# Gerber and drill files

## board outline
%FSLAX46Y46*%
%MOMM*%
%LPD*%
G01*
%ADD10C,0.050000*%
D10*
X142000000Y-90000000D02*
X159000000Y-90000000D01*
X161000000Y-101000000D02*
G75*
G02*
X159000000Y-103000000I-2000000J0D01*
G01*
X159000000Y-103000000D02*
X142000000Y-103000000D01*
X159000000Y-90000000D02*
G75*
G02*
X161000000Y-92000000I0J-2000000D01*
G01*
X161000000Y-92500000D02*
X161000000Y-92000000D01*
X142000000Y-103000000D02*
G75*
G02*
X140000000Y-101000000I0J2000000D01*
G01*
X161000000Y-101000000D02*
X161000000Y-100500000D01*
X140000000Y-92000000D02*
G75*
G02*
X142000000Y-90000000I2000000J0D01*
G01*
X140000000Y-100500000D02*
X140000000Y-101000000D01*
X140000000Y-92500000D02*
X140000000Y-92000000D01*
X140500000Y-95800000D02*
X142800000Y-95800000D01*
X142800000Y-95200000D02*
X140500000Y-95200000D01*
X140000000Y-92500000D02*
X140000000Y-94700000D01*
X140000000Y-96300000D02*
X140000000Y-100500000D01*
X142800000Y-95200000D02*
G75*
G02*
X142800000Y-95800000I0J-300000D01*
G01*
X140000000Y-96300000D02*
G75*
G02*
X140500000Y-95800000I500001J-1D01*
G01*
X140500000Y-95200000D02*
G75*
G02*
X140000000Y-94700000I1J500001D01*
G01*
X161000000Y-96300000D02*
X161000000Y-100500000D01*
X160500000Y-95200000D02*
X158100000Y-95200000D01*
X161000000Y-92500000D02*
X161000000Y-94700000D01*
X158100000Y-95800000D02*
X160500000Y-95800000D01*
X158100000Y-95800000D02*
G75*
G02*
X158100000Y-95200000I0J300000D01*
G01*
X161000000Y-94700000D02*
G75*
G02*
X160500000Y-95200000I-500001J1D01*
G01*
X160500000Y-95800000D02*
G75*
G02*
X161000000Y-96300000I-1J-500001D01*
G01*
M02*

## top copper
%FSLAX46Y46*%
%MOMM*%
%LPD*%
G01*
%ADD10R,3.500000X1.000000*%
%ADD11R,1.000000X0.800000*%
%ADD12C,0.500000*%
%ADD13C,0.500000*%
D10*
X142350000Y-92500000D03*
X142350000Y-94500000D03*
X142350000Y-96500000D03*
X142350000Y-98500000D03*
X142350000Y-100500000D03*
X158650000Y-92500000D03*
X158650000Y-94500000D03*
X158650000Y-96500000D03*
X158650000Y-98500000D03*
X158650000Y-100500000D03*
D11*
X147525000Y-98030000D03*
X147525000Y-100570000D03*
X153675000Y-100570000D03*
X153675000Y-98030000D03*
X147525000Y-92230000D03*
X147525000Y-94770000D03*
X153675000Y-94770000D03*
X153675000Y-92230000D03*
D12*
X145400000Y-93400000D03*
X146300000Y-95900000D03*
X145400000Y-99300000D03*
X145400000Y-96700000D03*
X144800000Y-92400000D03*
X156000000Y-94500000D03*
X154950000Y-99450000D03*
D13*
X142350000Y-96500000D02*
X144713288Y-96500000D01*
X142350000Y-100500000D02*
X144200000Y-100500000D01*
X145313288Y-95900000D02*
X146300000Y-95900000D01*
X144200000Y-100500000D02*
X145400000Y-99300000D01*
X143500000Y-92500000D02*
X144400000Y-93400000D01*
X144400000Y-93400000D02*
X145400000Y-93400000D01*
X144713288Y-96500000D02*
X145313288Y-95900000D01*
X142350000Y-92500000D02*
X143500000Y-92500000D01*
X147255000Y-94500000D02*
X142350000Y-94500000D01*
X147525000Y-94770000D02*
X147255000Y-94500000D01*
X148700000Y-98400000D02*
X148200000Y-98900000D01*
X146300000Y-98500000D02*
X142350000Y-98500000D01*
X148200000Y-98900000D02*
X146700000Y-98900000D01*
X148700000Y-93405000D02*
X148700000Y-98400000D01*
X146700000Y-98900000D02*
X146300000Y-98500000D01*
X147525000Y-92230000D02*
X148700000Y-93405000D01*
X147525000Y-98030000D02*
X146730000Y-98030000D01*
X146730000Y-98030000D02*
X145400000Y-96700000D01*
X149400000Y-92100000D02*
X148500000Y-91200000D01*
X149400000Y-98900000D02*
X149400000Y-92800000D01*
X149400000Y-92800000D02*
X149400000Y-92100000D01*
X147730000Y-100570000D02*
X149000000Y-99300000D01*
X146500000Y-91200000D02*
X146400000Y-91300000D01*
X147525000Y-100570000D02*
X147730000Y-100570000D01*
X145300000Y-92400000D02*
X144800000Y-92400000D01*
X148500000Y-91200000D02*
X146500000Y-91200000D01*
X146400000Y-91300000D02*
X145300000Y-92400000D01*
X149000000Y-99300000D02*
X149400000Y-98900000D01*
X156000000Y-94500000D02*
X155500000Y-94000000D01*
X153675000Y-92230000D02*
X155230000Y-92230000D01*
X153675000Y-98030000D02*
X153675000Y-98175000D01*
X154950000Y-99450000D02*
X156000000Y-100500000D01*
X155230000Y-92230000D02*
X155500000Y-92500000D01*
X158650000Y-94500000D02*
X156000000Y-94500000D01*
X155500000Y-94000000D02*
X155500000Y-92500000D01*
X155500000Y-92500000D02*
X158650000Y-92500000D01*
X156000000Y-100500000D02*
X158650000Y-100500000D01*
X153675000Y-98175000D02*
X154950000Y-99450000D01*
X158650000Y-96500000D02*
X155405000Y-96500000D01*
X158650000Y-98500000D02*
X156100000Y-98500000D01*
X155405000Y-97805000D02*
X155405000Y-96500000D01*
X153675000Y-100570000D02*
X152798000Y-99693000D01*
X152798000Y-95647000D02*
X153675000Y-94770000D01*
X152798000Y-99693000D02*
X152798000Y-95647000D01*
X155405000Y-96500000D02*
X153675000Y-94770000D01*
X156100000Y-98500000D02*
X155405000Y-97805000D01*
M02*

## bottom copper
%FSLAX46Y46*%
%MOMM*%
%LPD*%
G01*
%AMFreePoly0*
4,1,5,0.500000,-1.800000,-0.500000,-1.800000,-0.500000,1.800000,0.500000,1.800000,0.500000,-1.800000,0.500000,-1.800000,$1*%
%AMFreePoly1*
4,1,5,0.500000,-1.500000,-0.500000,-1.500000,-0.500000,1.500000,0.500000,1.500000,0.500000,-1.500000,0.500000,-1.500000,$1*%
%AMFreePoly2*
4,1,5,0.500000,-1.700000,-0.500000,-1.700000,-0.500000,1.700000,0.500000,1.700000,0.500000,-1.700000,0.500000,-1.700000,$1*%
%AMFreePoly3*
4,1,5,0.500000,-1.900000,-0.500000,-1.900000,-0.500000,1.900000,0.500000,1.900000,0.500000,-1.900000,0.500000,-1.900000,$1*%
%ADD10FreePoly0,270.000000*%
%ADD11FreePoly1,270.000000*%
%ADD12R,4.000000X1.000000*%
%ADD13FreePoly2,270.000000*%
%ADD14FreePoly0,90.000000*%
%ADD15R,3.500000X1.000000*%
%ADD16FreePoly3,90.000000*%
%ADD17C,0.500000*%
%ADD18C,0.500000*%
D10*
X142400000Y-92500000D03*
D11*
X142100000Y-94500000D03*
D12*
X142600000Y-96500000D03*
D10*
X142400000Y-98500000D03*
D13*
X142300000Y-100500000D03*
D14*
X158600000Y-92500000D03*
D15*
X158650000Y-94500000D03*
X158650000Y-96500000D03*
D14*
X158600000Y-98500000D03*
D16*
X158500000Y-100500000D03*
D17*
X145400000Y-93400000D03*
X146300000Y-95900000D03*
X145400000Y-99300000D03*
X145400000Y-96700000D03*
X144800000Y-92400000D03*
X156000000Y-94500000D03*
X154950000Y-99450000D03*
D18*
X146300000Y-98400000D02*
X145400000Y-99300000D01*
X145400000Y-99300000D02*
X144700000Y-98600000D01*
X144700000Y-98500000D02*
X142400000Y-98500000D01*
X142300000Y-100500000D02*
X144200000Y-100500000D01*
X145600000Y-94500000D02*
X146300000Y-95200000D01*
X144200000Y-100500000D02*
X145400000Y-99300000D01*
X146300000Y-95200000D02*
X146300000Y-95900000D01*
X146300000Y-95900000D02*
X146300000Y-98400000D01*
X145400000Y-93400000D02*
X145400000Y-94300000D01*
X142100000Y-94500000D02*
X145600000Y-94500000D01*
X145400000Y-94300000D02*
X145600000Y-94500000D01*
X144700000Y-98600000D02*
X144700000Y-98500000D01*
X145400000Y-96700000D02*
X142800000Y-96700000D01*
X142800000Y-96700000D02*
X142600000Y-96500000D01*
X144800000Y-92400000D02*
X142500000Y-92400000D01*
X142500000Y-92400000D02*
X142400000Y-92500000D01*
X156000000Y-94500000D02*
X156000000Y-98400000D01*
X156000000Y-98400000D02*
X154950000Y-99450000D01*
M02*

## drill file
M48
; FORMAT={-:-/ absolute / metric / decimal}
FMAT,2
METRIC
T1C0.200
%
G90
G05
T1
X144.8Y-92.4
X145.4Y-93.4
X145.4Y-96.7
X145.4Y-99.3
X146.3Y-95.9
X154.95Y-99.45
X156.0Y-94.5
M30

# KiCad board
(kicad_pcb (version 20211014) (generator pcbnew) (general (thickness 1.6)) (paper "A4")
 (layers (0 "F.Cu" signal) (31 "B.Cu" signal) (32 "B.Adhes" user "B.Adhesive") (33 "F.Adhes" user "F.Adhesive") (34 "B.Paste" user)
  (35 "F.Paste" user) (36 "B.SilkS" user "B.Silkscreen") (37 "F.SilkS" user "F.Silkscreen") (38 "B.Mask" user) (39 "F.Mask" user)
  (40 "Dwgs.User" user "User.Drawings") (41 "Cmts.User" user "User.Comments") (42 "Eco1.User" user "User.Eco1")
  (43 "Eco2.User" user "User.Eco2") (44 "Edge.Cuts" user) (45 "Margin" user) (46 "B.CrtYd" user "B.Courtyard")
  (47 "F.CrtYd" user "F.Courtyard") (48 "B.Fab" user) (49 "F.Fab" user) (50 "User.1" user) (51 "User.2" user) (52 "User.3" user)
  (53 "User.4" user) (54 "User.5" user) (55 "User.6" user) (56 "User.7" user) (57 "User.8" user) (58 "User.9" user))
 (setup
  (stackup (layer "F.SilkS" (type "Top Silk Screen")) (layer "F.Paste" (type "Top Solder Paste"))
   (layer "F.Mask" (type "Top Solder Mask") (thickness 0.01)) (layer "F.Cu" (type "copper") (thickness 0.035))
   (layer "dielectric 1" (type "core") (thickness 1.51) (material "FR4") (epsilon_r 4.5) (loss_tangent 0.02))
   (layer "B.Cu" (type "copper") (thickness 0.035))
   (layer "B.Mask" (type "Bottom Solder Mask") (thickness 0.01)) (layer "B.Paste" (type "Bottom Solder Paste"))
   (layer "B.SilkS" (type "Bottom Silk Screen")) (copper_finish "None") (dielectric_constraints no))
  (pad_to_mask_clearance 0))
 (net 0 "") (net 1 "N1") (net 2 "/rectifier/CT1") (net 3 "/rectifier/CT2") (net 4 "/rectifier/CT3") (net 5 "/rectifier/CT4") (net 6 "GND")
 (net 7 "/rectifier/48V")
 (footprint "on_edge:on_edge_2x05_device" (layer "F.Cu") (at 140 96.5 -90)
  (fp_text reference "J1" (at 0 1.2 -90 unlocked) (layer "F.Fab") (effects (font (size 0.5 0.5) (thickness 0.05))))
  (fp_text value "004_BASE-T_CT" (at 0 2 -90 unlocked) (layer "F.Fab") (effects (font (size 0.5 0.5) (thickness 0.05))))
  (fp_line (start -0.7 -0.5) (end -0.7 -2.8) (layer "Edge.Cuts") (width 0.05))
  (fp_line (start -1.3 -2.8) (end -1.3 -0.5) (layer "Edge.Cuts") (width 0.05))
  (fp_line (start -4 0) (end -1.8 0) (layer "Edge.Cuts") (width 0.05))
  (fp_line (start -0.2 0) (end 4 0) (layer "Edge.Cuts") (width 0.05))
  (fp_arc (start -1.3 -2.8) (mid -1 -3.1) (end -0.7 -2.8) (layer "Edge.Cuts") (width 0.05))
  (fp_arc (start -0.2 0) (mid -0.553553 -0.146447) (end -0.7 -0.5) (layer "Edge.Cuts") (width 0.05))
  (fp_arc (start -1.3 -0.5) (mid -1.446447 -0.146447) (end -1.8 0) (layer "Edge.Cuts") (width 0.05))
  (pad "1" smd rect (at -4 -2.35 90) (size 1 3.5) (layers "F.Cu" "F.Mask") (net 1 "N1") (zone_connect 0))
  (pad "2" smd rect (at -2 -2.35 270) (size 1 3.5) (layers "F.Cu" "F.Mask") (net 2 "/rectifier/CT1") (zone_connect 0))
  (pad "3" smd rect (at 0 -2.35 270) (size 1 3.5) (layers "F.Cu" "F.Mask") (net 1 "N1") (zone_connect 0))
  (pad "4" smd rect (at 2 -2.35 90) (size 1 3.5) (layers "F.Cu" "F.Mask") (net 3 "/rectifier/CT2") (zone_connect 0))
  (pad "5" smd rect (at 4 -2.35 90) (size 1 3.5) (layers "F.Cu" "F.Mask") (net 1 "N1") (zone_connect 0))
  (pad "6" smd custom (at -4 -2.4 270) (size 1 3.6) (layers "B.Cu" "B.Mask") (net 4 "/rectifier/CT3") (zone_connect 0)
   (options (clearance outline) (anchor rect)) (primitives))
  (pad "7" smd custom (at -2 -2.1 270) (size 1 3) (layers "B.Cu" "B.Mask") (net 1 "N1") (zone_connect 0)
   (options (clearance outline) (anchor rect)) (primitives))
  (pad "8" smd rect (at 0 -2.6 270) (size 1 4) (layers "B.Cu" "B.Mask") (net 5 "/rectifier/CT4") (zone_connect 0))
  (pad "9" smd custom (at 2 -2.4 270) (size 1 3.6) (layers "B.Cu" "B.Mask") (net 1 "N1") (zone_connect 0)
   (options (clearance outline) (anchor rect)) (primitives))
  (pad "10" smd custom (at 4 -2.3 270) (size 1 3.4) (layers "B.Cu" "B.Mask") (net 1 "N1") (zone_connect 0)
   (options (clearance outline) (anchor rect)) (primitives)))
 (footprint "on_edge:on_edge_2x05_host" (layer "F.Cu") (at 161 96.5 -90)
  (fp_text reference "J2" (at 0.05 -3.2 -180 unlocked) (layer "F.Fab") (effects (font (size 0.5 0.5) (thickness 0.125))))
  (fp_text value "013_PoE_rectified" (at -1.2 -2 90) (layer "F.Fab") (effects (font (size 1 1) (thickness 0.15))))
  (fp_line (start -0.2 0) (end 4 0) (layer "Edge.Cuts") (width 0.05))
  (fp_line (start -1.3 0.5) (end -1.3 2.9) (layer "Edge.Cuts") (width 0.05))
  (fp_line (start -4 0) (end -1.8 0) (layer "Edge.Cuts") (width 0.05))
  (fp_line (start -0.7 2.9) (end -0.7 0.5) (layer "Edge.Cuts") (width 0.05))
  (fp_arc (start -0.7 2.9) (mid -1 3.2) (end -1.3 2.9) (layer "Edge.Cuts") (width 0.05))
  (fp_arc (start -1.8 0) (mid -1.446447 0.146447) (end -1.3 0.5) (layer "Edge.Cuts") (width 0.05))
  (fp_arc (start -0.7 0.5) (mid -0.553553 0.146447) (end -0.2 0) (layer "Edge.Cuts") (width 0.05))
  (pad "1" smd rect (at -4 2.35 270) (size 1 3.5) (layers "F.Cu" "F.Mask") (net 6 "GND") (zone_connect 0))
  (pad "2" smd rect (at -2 2.35 270) (size 1 3.5) (layers "F.Cu" "F.Mask") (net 6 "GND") (zone_connect 0))
  (pad "3" smd rect (at 0 2.35 270) (size 1 3.5) (layers "F.Cu" "F.Mask") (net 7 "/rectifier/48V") (zone_connect 0))
  (pad "4" smd rect (at 2 2.35 270) (size 1 3.5) (layers "F.Cu" "F.Mask") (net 7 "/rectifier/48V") (zone_connect 0))
  (pad "5" smd rect (at 4 2.35 270) (size 1 3.5) (layers "F.Cu" "F.Mask") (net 6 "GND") (zone_connect 0))
  (pad "6" smd custom (at -4 2.4 90) (size 1 3.6) (layers "B.Cu" "B.Mask") (zone_connect 0) (options (clearance outline) (anchor rect))
   (primitives))
  (pad "7" smd rect (at -2 2.35 90) (size 1 3.5) (layers "B.Cu" "B.Mask") (zone_connect 0))
  (pad "8" smd rect (at 0 2.35 90) (size 1 3.5) (layers "B.Cu" "B.Mask") (zone_connect 0))
  (pad "9" smd custom (at 2 2.4 90) (size 1 3.6) (layers "B.Cu" "B.Mask") (zone_connect 0) (options (clearance outline) (anchor rect))
   (primitives))
  (pad "10" smd custom (at 4 2.5 90) (size 1 3.8) (layers "B.Cu" "B.Mask") (zone_connect 0) (options (clearance outline) (anchor rect))
   (primitives)))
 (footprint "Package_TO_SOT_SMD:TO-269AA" (layer "F.Cu") (at 150.6 99.3)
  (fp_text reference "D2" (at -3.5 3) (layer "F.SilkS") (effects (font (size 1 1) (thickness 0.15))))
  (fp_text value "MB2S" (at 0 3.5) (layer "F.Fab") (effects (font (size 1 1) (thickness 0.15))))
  (pad "1" smd rect (at -3.075 -1.27) (size 1 0.8) (layers "F.Cu" "F.Paste" "F.Mask") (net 5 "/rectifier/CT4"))
  (pad "2" smd rect (at -3.075 1.27) (size 1 0.8) (layers "F.Cu" "F.Paste" "F.Mask") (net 4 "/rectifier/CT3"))
  (pad "3" smd rect (at 3.075 1.27) (size 1 0.8) (layers "F.Cu" "F.Paste" "F.Mask") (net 7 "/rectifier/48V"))
  (pad "4" smd rect (at 3.075 -1.27) (size 1 0.8) (layers "F.Cu" "F.Paste" "F.Mask") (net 6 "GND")))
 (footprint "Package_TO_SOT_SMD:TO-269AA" (layer "F.Cu") (at 150.6 93.5)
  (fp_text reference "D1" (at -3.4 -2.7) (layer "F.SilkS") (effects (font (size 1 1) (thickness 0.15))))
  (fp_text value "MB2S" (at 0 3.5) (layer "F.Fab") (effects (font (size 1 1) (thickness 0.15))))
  (pad "1" smd rect (at -3.075 -1.27) (size 1 0.8) (layers "F.Cu" "F.Paste" "F.Mask") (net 3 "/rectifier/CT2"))
  (pad "2" smd rect (at -3.075 1.27) (size 1 0.8) (layers "F.Cu" "F.Paste" "F.Mask") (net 2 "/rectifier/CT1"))
  (pad "3" smd rect (at 3.075 1.27) (size 1 0.8) (layers "F.Cu" "F.Paste" "F.Mask") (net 7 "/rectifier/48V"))
  (pad "4" smd rect (at 3.075 -1.27) (size 1 0.8) (layers "F.Cu" "F.Paste" "F.Mask") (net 6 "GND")))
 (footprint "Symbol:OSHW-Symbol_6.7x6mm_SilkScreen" (layer "B.Cu") (at 150 99 180)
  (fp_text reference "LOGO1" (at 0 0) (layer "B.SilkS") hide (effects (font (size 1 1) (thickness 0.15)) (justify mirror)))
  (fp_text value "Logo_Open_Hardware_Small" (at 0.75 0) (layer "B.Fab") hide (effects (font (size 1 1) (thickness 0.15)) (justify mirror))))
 (gr_line (start 142 90) (end 159 90) (layer "Edge.Cuts") (width 0.05))
 (gr_arc (start 161 101) (mid 160.414214 102.414214) (end 159 103) (layer "Edge.Cuts") (width 0.05))
 (gr_line (start 159 103) (end 142 103) (layer "Edge.Cuts") (width 0.05))
 (gr_arc (start 159 90) (mid 160.414214 90.585786) (end 161 92) (layer "Edge.Cuts") (width 0.05))
 (gr_line (start 161 92.5) (end 161 92) (layer "Edge.Cuts") (width 0.05))
 (gr_arc (start 142 103) (mid 140.585786 102.414214) (end 140 101) (layer "Edge.Cuts") (width 0.05))
 (gr_line (start 161 101) (end 161 100.5) (layer "Edge.Cuts") (width 0.05))
 (gr_arc (start 140 92) (mid 140.585786 90.585786) (end 142 90) (layer "Edge.Cuts") (width 0.05))
 (gr_line (start 140 100.5) (end 140 101) (layer "Edge.Cuts") (width 0.05))
 (gr_line (start 140 92.5) (end 140 92) (layer "Edge.Cuts") (width 0.05))
 (segment (start 142.35 96.5) (end 144.713288 96.5) (width 0.5) (layer "F.Cu") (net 1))
 (segment (start 142.35 100.5) (end 144.2 100.5) (width 0.5) (layer "F.Cu") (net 1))
 (segment (start 145.313288 95.9) (end 146.3 95.9) (width 0.5) (layer "F.Cu") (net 1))
 (segment (start 144.2 100.5) (end 145.4 99.3) (width 0.5) (layer "F.Cu") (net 1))
 (segment (start 143.5 92.5) (end 144.4 93.4) (width 0.5) (layer "F.Cu") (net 1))
 (segment (start 144.4 93.4) (end 145.4 93.4) (width 0.5) (layer "F.Cu") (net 1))
 (segment (start 144.713288 96.5) (end 145.313288 95.9) (width 0.5) (layer "F.Cu") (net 1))
 (segment (start 142.35 92.5) (end 143.5 92.5) (width 0.5) (layer "F.Cu") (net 1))
 (via (at 145.4 93.4) (size 0.5) (drill 0.2) (layers "F.Cu" "B.Cu") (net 1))
 (via (at 146.3 95.9) (size 0.5) (drill 0.2) (layers "F.Cu" "B.Cu") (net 1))
 (via (at 145.4 99.3) (size 0.5) (drill 0.2) (layers "F.Cu" "B.Cu") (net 1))
 (segment (start 146.3 98.4) (end 145.4 99.3) (width 0.5) (layer "B.Cu") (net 1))
 (segment (start 145.4 99.3) (end 144.7 98.6) (width 0.5) (layer "B.Cu") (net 1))
 (segment (start 144.7 98.5) (end 142.4 98.5) (width 0.5) (layer "B.Cu") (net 1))
 (segment (start 142.3 100.5) (end 144.2 100.5) (width 0.5) (layer "B.Cu") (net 1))
 (segment (start 145.6 94.5) (end 146.3 95.2) (width 0.5) (layer "B.Cu") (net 1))
 (segment (start 144.2 100.5) (end 145.4 99.3) (width 0.5) (layer "B.Cu") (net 1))
 (segment (start 146.3 95.2) (end 146.3 95.9) (width 0.5) (layer "B.Cu") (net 1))
 (segment (start 146.3 95.9) (end 146.3 98.4) (width 0.5) (layer "B.Cu") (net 1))
 (segment (start 145.4 93.4) (end 145.4 94.3) (width 0.5) (layer "B.Cu") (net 1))
 (segment (start 142.1 94.5) (end 145.6 94.5) (width 0.5) (layer "B.Cu") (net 1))
 (segment (start 145.4 94.3) (end 145.6 94.5) (width 0.5) (layer "B.Cu") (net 1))
 (segment (start 144.7 98.6) (end 144.7 98.5) (width 0.5) (layer "B.Cu") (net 1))
 (segment (start 147.255 94.5) (end 142.35 94.5) (width 0.5) (layer "F.Cu") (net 2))
 (segment (start 147.525 94.77) (end 147.255 94.5) (width 0.5) (layer "F.Cu") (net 2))
 (segment (start 148.7 98.4) (end 148.2 98.9) (width 0.5) (layer "F.Cu") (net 3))
 (segment (start 146.3 98.5) (end 142.35 98.5) (width 0.5) (layer "F.Cu") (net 3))
 (segment (start 148.2 98.9) (end 146.7 98.9) (width 0.5) (layer "F.Cu") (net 3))
 (segment (start 148.7 93.405) (end 148.7 98.4) (width 0.5) (layer "F.Cu") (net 3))
 (segment (start 146.7 98.9) (end 146.3 98.5) (width 0.5) (layer "F.Cu") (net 3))
 (segment (start 147.525 92.23) (end 148.7 93.405) (width 0.5) (layer "F.Cu") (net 3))
 (segment (start 147.525 98.03) (end 146.73 98.03) (width 0.5) (layer "F.Cu") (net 5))
 (segment (start 146.73 98.03) (end 145.4 96.7) (width 0.5) (layer "F.Cu") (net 5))
 (via (at 145.4 96.7) (size 0.5) (drill 0.2) (layers "F.Cu" "B.Cu") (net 5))
 (segment (start 145.4 96.7) (end 142.8 96.7) (width 0.5) (layer "B.Cu") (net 5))
 (segment (start 142.8 96.7) (end 142.6 96.5) (width 0.5) (layer "B.Cu") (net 5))
 (segment (start 149.4 92.1) (end 148.5 91.2) (width 0.5) (layer "F.Cu") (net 4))
 (segment (start 149.4 98.9) (end 149.4 92.8) (width 0.5) (layer "F.Cu") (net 4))
 (segment (start 149.4 92.8) (end 149.4 92.1) (width 0.5) (layer "F.Cu") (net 4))
 (segment (start 147.73 100.57) (end 149 99.3) (width 0.5) (layer "F.Cu") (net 4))
 (segment (start 146.5 91.2) (end 146.4 91.3) (width 0.5) (layer "F.Cu") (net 4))
 (segment (start 147.525 100.57) (end 147.73 100.57) (width 0.5) (layer "F.Cu") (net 4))
 (segment (start 145.3 92.4) (end 144.8 92.4) (width 0.5) (layer "F.Cu") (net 4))
 (segment (start 148.5 91.2) (end 146.5 91.2) (width 0.5) (layer "F.Cu") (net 4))
 (segment (start 146.4 91.3) (end 145.3 92.4) (width 0.5) (layer "F.Cu") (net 4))
 (segment (start 149 99.3) (end 149.4 98.9) (width 0.5) (layer "F.Cu") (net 4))
 (via (at 144.8 92.4) (size 0.5) (drill 0.2) (layers "F.Cu" "B.Cu") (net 4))
 (segment (start 144.8 92.4) (end 142.5 92.4) (width 0.5) (layer "B.Cu") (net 4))
 (segment (start 142.5 92.4) (end 142.4 92.5) (width 0.5) (layer "B.Cu") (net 4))
 (segment (start 156 94.5) (end 155.5 94) (width 0.5) (layer "F.Cu") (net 6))
 (segment (start 153.675 92.23) (end 155.23 92.23) (width 0.5) (layer "F.Cu") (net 6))
 (segment (start 153.675 98.03) (end 153.675 98.175) (width 0.5) (layer "F.Cu") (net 6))
 (segment (start 154.95 99.45) (end 156 100.5) (width 0.5) (layer "F.Cu") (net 6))
 (segment (start 155.23 92.23) (end 155.5 92.5) (width 0.5) (layer "F.Cu") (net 6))
 (segment (start 158.65 94.5) (end 156 94.5) (width 0.5) (layer "F.Cu") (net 6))
 (segment (start 155.5 94) (end 155.5 92.5) (width 0.5) (layer "F.Cu") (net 6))
 (segment (start 155.5 92.5) (end 158.65 92.5) (width 0.5) (layer "F.Cu") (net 6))
 (segment (start 156 100.5) (end 158.65 100.5) (width 0.5) (layer "F.Cu") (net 6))
 (segment (start 153.675 98.175) (end 154.95 99.45) (width 0.5) (layer "F.Cu") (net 6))
 (via (at 156 94.5) (size 0.5) (drill 0.2) (layers "F.Cu" "B.Cu") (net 6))
 (via (at 154.95 99.45) (size 0.5) (drill 0.2) (layers "F.Cu" "B.Cu") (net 6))
 (segment (start 156 94.5) (end 156 98.4) (width 0.5) (layer "B.Cu") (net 6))
 (segment (start 156 98.4) (end 154.95 99.45) (width 0.5) (layer "B.Cu") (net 6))
 (segment (start 158.65 96.5) (end 155.405 96.5) (width 0.5) (layer "F.Cu") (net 7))
 (segment (start 158.65 98.5) (end 156.1 98.5) (width 0.5) (layer "F.Cu") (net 7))
 (segment (start 155.405 97.805) (end 155.405 96.5) (width 0.5) (layer "F.Cu") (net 7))
 (segment (start 153.675 100.57) (end 152.798 99.693) (width 0.5) (layer "F.Cu") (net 7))
 (segment (start 152.798 95.647) (end 153.675 94.77) (width 0.5) (layer "F.Cu") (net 7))
 (segment (start 152.798 99.693) (end 152.798 95.647) (width 0.5) (layer "F.Cu") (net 7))
 (segment (start 155.405 96.5) (end 153.675 94.77) (width 0.5) (layer "F.Cu") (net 7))
 (segment (start 156.1 98.5) (end 155.405 97.805) (width 0.5) (layer "F.Cu") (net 7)))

